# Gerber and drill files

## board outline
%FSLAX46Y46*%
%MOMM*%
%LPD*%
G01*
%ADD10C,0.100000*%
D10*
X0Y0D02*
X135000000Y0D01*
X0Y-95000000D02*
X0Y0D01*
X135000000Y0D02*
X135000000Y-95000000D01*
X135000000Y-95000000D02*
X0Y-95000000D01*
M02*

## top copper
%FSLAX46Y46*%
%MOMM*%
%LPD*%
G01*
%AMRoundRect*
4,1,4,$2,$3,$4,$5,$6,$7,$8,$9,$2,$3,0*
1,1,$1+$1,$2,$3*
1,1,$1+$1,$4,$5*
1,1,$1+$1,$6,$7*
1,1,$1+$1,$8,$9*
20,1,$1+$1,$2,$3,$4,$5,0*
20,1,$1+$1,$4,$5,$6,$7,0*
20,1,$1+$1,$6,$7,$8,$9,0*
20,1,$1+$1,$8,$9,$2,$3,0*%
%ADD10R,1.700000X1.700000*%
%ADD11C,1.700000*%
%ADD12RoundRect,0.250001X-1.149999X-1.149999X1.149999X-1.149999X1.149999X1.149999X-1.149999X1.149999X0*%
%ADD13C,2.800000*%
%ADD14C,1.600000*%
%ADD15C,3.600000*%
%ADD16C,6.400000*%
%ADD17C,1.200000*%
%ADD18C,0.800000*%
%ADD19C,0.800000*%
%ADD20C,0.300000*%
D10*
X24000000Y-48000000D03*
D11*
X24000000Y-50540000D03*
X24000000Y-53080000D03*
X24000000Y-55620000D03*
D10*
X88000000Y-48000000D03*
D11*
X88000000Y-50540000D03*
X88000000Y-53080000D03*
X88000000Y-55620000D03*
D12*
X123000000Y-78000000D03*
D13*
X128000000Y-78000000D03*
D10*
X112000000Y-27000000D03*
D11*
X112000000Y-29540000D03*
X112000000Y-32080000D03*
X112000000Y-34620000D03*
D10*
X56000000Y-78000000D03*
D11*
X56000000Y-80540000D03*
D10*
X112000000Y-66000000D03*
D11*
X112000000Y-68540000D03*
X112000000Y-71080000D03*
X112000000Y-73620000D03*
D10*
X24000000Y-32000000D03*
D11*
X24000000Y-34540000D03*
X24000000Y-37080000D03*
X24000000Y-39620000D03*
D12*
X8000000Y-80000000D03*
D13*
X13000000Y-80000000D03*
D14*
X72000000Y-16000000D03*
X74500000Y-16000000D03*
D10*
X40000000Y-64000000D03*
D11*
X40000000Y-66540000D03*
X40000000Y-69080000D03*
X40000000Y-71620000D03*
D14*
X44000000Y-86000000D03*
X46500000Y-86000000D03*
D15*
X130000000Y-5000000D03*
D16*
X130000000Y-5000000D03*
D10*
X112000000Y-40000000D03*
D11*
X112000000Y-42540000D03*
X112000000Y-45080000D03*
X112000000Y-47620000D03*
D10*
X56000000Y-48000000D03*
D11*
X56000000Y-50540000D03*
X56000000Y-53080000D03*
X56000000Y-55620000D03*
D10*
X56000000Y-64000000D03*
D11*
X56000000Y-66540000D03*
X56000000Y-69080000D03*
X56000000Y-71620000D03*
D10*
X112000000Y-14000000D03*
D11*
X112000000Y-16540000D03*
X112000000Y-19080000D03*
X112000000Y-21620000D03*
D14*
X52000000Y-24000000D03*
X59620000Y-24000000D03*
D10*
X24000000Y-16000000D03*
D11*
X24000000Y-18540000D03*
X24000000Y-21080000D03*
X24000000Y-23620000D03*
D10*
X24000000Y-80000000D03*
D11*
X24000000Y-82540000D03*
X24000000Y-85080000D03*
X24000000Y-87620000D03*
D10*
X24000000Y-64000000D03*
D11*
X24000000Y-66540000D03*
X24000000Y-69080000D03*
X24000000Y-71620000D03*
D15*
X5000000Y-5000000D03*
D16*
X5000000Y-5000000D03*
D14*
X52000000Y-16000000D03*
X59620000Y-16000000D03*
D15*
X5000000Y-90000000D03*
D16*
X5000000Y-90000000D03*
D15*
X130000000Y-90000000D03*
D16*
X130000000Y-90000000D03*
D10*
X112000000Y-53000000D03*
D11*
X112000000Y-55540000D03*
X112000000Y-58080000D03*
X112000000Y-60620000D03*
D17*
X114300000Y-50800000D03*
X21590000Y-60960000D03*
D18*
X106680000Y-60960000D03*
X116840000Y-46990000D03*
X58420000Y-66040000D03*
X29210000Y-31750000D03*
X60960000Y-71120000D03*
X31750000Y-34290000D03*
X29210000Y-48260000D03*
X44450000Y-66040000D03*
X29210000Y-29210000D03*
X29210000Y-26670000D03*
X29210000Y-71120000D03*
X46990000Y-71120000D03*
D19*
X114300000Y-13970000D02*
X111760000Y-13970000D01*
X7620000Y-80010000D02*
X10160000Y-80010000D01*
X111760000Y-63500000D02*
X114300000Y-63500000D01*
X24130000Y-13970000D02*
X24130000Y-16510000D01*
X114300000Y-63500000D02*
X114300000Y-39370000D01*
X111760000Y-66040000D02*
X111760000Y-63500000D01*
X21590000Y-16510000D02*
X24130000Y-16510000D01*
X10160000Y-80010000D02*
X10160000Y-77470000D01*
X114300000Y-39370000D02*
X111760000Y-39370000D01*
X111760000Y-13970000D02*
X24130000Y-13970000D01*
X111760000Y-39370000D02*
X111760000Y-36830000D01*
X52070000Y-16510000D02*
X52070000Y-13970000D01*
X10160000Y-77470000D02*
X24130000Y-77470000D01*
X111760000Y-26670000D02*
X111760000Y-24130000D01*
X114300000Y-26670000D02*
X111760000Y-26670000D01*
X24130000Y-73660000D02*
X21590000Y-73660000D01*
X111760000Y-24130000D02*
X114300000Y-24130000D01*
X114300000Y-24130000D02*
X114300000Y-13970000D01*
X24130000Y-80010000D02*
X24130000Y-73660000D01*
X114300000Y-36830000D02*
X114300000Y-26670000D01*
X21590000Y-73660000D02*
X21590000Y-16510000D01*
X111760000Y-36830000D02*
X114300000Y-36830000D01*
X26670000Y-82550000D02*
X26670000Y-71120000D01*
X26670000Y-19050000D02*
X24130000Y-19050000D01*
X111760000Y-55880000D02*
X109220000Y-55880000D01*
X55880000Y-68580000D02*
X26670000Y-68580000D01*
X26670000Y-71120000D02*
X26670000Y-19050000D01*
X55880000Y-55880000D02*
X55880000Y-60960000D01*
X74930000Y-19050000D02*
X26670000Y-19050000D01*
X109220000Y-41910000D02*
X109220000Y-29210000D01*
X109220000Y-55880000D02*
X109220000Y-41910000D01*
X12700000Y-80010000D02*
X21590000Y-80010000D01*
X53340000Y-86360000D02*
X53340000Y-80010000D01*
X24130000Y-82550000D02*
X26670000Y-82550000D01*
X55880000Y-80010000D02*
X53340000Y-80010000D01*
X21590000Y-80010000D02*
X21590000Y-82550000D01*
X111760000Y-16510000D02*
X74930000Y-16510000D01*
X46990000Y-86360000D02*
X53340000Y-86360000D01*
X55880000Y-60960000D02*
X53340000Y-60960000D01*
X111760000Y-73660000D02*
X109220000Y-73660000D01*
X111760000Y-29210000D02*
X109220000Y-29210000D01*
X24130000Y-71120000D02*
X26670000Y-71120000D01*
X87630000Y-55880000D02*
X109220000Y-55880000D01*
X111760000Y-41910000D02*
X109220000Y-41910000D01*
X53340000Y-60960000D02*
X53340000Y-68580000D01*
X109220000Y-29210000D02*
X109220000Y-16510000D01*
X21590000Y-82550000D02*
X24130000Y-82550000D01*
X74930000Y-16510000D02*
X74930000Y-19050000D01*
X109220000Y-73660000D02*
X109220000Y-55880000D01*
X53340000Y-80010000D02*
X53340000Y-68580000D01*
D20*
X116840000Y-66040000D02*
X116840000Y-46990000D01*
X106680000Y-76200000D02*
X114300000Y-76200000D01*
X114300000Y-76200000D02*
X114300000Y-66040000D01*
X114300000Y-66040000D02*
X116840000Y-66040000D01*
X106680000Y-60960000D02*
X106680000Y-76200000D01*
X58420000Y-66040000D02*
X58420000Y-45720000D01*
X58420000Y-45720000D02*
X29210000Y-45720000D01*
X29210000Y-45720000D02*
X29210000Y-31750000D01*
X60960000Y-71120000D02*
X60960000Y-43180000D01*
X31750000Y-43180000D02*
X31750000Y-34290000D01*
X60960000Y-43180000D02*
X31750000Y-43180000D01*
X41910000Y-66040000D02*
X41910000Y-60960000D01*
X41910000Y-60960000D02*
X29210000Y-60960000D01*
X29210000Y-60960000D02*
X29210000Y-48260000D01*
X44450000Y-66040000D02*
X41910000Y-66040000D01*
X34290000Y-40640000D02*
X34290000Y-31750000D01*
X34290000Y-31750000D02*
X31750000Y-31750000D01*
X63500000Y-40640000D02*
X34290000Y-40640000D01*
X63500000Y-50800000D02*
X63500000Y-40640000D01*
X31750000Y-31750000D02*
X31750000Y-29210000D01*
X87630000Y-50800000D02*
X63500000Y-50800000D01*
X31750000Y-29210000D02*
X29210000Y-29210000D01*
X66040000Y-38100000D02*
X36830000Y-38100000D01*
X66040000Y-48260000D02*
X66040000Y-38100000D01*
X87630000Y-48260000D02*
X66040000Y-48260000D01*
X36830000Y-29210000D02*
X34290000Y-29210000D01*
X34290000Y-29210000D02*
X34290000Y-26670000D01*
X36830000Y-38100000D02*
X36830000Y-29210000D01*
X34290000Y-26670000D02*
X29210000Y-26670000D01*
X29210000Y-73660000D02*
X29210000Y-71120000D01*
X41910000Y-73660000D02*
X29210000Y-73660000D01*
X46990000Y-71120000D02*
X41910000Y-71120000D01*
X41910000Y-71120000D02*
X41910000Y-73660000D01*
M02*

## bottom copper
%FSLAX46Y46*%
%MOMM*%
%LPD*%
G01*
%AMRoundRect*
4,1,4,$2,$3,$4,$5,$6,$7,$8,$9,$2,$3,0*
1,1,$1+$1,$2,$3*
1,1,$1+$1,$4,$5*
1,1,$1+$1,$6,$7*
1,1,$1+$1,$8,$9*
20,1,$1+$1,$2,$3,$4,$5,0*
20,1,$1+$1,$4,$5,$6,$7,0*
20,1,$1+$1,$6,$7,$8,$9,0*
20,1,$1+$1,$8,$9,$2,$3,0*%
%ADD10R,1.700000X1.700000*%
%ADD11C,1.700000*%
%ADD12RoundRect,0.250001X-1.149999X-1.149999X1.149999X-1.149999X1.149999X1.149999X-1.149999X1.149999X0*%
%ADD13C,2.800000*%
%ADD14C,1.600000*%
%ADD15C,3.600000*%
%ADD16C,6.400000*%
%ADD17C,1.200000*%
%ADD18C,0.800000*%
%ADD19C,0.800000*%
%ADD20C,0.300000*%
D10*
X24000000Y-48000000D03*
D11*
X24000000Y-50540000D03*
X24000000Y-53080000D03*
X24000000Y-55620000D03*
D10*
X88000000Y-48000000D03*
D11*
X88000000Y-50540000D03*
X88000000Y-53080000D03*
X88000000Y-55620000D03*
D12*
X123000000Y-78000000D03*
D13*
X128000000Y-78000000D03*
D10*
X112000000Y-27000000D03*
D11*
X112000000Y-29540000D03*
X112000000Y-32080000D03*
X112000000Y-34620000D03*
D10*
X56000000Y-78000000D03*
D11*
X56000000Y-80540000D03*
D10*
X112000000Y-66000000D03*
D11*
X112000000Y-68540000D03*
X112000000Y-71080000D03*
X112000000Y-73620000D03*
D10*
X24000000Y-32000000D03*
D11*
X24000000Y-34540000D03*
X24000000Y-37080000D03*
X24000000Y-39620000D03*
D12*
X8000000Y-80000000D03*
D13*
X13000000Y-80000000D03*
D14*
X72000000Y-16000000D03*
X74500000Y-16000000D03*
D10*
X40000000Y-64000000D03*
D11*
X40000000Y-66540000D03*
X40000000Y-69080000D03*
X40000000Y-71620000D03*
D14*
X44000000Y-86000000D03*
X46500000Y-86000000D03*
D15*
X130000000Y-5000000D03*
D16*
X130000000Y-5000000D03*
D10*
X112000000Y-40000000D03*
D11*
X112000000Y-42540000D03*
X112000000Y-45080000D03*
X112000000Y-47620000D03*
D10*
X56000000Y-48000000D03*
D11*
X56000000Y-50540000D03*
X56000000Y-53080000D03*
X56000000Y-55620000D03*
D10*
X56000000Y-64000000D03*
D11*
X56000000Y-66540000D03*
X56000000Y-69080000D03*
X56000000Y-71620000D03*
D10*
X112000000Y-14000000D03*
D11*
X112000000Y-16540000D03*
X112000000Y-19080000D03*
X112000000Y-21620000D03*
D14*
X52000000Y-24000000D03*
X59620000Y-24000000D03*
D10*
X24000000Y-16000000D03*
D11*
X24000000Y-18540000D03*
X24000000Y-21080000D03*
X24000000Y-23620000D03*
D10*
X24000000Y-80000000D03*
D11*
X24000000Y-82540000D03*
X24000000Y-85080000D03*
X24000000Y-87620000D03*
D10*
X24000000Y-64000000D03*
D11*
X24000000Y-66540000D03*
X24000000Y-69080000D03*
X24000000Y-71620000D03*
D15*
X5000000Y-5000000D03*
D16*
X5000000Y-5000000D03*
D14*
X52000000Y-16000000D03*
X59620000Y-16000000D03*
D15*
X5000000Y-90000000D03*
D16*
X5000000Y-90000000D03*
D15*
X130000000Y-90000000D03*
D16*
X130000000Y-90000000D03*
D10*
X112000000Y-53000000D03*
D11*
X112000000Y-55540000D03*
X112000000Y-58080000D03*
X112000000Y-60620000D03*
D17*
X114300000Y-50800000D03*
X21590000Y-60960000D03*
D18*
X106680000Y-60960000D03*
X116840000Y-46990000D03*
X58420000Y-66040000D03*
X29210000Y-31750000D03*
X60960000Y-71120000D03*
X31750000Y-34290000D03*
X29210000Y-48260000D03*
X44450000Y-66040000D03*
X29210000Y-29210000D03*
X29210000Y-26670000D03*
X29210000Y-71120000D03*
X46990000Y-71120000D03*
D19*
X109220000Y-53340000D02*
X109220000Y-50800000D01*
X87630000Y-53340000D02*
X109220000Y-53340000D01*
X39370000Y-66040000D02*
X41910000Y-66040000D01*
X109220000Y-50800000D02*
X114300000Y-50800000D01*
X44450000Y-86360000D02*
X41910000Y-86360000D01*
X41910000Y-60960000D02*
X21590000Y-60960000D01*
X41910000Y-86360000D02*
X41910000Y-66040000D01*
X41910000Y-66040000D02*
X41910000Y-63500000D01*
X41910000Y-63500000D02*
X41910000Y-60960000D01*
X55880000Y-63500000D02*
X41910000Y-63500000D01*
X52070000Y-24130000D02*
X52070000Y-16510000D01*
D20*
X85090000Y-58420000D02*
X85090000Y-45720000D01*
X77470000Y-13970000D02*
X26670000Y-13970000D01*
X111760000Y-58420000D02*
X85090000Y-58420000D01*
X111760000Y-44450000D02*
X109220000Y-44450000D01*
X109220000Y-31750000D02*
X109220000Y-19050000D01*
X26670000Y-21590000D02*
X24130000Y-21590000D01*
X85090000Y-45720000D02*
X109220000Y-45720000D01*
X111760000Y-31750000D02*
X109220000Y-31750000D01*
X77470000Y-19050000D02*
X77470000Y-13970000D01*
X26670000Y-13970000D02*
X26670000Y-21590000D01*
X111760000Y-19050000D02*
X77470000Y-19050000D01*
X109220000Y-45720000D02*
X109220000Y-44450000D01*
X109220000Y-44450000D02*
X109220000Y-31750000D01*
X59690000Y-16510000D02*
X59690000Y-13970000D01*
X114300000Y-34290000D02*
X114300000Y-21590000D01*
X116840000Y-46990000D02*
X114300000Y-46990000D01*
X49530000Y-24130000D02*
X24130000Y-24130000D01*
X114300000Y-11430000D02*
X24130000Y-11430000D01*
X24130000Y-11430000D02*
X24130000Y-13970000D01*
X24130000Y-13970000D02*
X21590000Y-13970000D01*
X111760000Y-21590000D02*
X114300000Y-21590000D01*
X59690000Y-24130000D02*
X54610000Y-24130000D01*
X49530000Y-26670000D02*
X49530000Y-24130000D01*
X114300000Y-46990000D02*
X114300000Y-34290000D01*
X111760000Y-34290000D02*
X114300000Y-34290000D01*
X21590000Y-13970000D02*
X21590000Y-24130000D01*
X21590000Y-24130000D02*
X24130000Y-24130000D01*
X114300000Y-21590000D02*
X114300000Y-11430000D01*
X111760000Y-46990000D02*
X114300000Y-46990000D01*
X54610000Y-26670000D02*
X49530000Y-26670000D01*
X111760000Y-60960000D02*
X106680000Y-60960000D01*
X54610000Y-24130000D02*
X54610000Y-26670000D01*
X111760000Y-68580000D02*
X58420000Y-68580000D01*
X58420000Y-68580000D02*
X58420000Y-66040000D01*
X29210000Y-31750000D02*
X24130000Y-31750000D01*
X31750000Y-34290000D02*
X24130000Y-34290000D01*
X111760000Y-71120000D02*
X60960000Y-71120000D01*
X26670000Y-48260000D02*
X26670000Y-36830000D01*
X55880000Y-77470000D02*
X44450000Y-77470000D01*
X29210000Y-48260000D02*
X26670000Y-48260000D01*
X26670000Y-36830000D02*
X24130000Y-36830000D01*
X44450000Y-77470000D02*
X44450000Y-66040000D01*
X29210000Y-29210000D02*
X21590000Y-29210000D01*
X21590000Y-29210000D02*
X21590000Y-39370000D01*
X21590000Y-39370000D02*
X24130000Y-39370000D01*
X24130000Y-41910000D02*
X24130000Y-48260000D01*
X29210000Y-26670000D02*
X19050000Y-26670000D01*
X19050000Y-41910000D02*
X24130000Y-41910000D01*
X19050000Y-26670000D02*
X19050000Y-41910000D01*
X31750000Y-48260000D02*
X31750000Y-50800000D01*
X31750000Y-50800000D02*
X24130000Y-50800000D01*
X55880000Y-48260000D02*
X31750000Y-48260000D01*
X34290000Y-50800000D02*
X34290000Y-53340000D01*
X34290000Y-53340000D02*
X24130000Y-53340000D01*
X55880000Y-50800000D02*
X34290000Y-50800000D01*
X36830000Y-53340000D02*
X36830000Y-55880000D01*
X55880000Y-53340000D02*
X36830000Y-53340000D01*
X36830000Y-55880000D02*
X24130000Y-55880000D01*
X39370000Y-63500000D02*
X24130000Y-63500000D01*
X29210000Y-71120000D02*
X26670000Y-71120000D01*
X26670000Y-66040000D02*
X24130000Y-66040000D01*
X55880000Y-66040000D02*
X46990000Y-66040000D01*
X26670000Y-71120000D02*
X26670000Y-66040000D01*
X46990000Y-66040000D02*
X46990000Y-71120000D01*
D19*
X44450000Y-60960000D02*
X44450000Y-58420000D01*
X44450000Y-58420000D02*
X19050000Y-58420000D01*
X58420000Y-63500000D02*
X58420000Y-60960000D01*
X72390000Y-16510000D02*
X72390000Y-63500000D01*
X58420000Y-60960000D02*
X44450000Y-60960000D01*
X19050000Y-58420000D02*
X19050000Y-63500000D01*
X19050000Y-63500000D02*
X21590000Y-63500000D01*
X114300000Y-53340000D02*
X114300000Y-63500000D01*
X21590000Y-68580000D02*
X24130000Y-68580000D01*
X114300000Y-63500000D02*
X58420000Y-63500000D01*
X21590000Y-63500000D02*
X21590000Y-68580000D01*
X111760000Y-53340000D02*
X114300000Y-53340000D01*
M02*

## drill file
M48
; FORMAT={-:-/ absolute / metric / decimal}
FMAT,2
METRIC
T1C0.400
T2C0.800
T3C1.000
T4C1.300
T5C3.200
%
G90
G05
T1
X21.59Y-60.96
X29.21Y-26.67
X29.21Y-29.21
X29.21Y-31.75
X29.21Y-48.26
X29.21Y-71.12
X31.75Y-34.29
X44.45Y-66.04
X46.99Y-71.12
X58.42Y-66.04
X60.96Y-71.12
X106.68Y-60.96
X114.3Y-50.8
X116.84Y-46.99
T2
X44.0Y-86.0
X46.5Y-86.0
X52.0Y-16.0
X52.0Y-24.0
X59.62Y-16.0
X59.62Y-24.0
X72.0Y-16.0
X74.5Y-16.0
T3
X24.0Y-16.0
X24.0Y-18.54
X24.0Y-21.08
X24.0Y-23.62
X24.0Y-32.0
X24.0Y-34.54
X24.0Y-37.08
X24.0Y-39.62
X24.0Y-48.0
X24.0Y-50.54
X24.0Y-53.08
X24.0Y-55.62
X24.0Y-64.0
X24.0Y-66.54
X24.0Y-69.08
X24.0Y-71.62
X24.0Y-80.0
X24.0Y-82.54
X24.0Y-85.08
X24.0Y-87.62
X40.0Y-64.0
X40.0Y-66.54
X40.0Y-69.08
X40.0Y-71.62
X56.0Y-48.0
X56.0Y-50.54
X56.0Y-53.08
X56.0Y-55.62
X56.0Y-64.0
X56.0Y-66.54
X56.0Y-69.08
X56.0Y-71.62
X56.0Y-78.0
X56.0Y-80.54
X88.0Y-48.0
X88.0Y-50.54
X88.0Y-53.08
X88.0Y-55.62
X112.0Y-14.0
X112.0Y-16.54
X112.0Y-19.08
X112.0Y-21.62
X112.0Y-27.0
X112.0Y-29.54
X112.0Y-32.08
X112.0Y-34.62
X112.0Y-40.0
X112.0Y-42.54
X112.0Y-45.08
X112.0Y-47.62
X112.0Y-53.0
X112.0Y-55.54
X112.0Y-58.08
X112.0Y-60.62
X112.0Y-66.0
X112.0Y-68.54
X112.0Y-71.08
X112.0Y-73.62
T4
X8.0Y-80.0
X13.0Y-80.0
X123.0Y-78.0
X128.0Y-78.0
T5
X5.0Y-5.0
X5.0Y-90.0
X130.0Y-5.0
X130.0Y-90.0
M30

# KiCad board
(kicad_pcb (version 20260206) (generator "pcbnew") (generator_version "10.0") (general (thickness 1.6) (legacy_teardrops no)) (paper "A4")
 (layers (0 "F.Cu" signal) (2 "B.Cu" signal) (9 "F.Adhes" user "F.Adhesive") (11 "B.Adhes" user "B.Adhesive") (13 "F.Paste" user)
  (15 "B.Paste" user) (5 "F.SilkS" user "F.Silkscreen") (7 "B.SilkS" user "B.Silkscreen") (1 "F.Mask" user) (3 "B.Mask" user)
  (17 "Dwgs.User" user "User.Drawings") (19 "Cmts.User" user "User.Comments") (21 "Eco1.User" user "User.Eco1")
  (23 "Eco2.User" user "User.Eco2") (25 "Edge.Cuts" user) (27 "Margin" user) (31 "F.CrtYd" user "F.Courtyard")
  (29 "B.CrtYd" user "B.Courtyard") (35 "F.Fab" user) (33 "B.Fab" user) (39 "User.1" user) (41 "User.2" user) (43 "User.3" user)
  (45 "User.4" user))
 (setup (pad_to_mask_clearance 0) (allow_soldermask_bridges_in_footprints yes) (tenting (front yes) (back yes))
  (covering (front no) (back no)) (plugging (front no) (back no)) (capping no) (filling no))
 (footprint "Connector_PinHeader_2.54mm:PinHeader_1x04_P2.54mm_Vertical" (layer "F.Cu") (at 24 48)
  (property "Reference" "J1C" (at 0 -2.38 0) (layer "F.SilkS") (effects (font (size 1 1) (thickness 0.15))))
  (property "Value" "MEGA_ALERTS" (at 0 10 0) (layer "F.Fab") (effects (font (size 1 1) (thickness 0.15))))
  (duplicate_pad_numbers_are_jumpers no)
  (pad "1" thru_hole rect (at 0 0) (size 1.7 1.7) (drill 1) (layers "*.Cu" "*.Mask") (remove_unused_layers no) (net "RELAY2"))
  (pad "2" thru_hole circle (at 0 2.54) (size 1.7 1.7) (drill 1) (layers "*.Cu" "*.Mask") (remove_unused_layers no) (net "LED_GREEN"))
  (pad "3" thru_hole circle (at 0 5.08) (size 1.7 1.7) (drill 1) (layers "*.Cu" "*.Mask") (remove_unused_layers no) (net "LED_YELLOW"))
  (pad "4" thru_hole circle (at 0 7.62) (size 1.7 1.7) (drill 1) (layers "*.Cu" "*.Mask") (remove_unused_layers no) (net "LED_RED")))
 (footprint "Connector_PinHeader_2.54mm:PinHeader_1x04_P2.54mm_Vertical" (layer "F.Cu") (at 88 48)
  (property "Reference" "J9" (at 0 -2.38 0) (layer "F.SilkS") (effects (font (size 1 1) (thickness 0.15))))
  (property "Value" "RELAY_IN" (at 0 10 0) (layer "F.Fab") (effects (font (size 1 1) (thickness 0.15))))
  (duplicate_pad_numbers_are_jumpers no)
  (pad "1" thru_hole rect (at 0 0) (size 1.7 1.7) (drill 1) (layers "*.Cu" "*.Mask") (remove_unused_layers no) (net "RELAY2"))
  (pad "2" thru_hole circle (at 0 2.54) (size 1.7 1.7) (drill 1) (layers "*.Cu" "*.Mask") (remove_unused_layers no) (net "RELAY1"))
  (pad "3" thru_hole circle (at 0 5.08) (size 1.7 1.7) (drill 1) (layers "*.Cu" "*.Mask") (remove_unused_layers no) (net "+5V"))
  (pad "4" thru_hole circle (at 0 7.62) (size 1.7 1.7) (drill 1) (layers "*.Cu" "*.Mask") (remove_unused_layers no) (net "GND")))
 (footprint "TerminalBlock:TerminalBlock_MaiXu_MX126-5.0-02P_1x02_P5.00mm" (layer "F.Cu") (at 123 78)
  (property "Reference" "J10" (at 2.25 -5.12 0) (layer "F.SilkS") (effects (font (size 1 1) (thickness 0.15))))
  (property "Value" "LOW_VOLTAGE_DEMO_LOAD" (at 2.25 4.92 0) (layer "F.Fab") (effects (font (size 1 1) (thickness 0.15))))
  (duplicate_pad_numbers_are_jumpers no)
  (pad "1" thru_hole roundrect (at 0 0) (size 2.8 2.8) (drill 1.3) (layers "*.Cu" "*.Mask") (remove_unused_layers no)
   (roundrect_rratio 0.089286) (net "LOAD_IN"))
  (pad "2" thru_hole circle (at 5 0) (size 2.8 2.8) (drill 1.3) (layers "*.Cu" "*.Mask") (remove_unused_layers no) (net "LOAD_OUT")))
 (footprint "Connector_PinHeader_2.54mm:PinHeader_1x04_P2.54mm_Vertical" (layer "F.Cu") (at 112 27)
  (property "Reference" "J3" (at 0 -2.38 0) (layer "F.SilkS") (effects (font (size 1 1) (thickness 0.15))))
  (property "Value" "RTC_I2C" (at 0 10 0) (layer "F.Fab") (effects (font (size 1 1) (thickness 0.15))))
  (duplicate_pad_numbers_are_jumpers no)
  (pad "1" thru_hole rect (at 0 0) (size 1.7 1.7) (drill 1) (layers "*.Cu" "*.Mask") (remove_unused_layers no) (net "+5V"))
  (pad "2" thru_hole circle (at 0 2.54) (size 1.7 1.7) (drill 1) (layers "*.Cu" "*.Mask") (remove_unused_layers no) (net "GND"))
  (pad "3" thru_hole circle (at 0 5.08) (size 1.7 1.7) (drill 1) (layers "*.Cu" "*.Mask") (remove_unused_layers no) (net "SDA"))
  (pad "4" thru_hole circle (at 0 7.62) (size 1.7 1.7) (drill 1) (layers "*.Cu" "*.Mask") (remove_unused_layers no) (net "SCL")))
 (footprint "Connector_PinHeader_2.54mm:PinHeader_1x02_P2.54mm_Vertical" (layer "F.Cu") (at 56 78)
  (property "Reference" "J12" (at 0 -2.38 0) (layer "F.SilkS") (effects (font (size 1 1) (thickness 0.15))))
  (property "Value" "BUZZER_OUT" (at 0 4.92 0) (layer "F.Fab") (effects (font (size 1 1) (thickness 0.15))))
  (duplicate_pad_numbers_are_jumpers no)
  (pad "1" thru_hole rect (at 0 0) (size 1.7 1.7) (drill 1) (layers "*.Cu" "*.Mask") (remove_unused_layers no) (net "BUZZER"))
  (pad "2" thru_hole circle (at 0 2.54) (size 1.7 1.7) (drill 1) (layers "*.Cu" "*.Mask") (remove_unused_layers no) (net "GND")))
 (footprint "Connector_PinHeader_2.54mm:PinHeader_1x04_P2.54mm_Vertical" (layer "F.Cu") (at 112 66)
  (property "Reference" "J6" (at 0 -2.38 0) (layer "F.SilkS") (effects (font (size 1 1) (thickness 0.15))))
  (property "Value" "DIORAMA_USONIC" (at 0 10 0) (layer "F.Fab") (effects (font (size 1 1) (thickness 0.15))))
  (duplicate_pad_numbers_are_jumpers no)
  (pad "1" thru_hole rect (at 0 0) (size 1.7 1.7) (drill 1) (layers "*.Cu" "*.Mask") (remove_unused_layers no) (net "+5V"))
  (pad "2" thru_hole circle (at 0 2.54) (size 1.7 1.7) (drill 1) (layers "*.Cu" "*.Mask") (remove_unused_layers no) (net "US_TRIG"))
  (pad "3" thru_hole circle (at 0 5.08) (size 1.7 1.7) (drill 1) (layers "*.Cu" "*.Mask") (remove_unused_layers no) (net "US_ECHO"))
  (pad "4" thru_hole circle (at 0 7.62) (size 1.7 1.7) (drill 1) (layers "*.Cu" "*.Mask") (remove_unused_layers no) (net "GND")))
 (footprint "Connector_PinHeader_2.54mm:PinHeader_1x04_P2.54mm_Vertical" (layer "F.Cu") (at 24 32)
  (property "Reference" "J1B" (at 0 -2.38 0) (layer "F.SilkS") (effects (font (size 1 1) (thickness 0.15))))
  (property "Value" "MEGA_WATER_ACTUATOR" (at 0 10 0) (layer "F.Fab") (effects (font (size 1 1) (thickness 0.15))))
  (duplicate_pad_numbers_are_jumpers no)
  (pad "1" thru_hole rect (at 0 0) (size 1.7 1.7) (drill 1) (layers "*.Cu" "*.Mask") (remove_unused_layers no) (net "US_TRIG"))
  (pad "2" thru_hole circle (at 0 2.54) (size 1.7 1.7) (drill 1) (layers "*.Cu" "*.Mask") (remove_unused_layers no) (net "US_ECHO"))
  (pad "3" thru_hole circle (at 0 5.08) (size 1.7 1.7) (drill 1) (layers "*.Cu" "*.Mask") (remove_unused_layers no) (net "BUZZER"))
  (pad "4" thru_hole circle (at 0 7.62) (size 1.7 1.7) (drill 1) (layers "*.Cu" "*.Mask") (remove_unused_layers no) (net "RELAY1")))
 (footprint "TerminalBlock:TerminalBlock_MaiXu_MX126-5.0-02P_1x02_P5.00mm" (layer "F.Cu") (at 8 80)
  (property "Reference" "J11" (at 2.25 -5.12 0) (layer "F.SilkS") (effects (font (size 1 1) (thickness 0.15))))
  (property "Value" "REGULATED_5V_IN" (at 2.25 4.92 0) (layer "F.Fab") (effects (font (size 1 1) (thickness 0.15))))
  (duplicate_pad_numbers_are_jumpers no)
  (pad "1" thru_hole roundrect (at 0 0) (size 2.8 2.8) (drill 1.3) (layers "*.Cu" "*.Mask") (remove_unused_layers no)
   (roundrect_rratio 0.089286) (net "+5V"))
  (pad "2" thru_hole circle (at 5 0) (size 2.8 2.8) (drill 1.3) (layers "*.Cu" "*.Mask") (remove_unused_layers no) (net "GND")))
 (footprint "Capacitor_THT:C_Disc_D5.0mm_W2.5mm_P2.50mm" (layer "F.Cu") (at 72 16)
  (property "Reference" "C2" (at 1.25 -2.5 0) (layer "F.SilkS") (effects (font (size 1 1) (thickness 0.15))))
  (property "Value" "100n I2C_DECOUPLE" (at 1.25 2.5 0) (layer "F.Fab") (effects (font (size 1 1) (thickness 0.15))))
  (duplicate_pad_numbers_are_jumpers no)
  (pad "1" thru_hole circle (at 0 0) (size 1.6 1.6) (drill 0.8) (layers "*.Cu" "*.Mask") (remove_unused_layers no) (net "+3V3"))
  (pad "2" thru_hole circle (at 2.5 0) (size 1.6 1.6) (drill 0.8) (layers "*.Cu" "*.Mask") (remove_unused_layers no) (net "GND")))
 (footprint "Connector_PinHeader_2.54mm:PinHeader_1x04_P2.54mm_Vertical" (layer "F.Cu") (at 40 64)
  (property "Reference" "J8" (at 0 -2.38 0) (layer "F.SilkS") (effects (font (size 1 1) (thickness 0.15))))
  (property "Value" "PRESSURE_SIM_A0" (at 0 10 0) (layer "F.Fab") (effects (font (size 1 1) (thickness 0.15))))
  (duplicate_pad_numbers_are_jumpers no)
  (pad "1" thru_hole rect (at 0 0) (size 1.7 1.7) (drill 1) (layers "*.Cu" "*.Mask") (remove_unused_layers no) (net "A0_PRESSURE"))
  (pad "2" thru_hole circle (at 0 2.54) (size 1.7 1.7) (drill 1) (layers "*.Cu" "*.Mask") (remove_unused_layers no) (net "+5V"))
  (pad "3" thru_hole circle (at 0 5.08) (size 1.7 1.7) (drill 1) (layers "*.Cu" "*.Mask") (remove_unused_layers no) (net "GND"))
  (pad "4" thru_hole circle (at 0 7.62) (size 1.7 1.7) (drill 1) (layers "*.Cu" "*.Mask") (remove_unused_layers no)))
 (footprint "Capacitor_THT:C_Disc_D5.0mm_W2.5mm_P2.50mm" (layer "F.Cu") (at 44 86)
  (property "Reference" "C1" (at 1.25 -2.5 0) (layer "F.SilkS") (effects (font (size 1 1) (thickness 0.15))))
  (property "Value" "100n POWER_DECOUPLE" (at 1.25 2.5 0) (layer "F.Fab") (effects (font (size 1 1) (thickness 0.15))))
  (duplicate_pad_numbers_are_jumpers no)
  (pad "1" thru_hole circle (at 0 0) (size 1.6 1.6) (drill 0.8) (layers "*.Cu" "*.Mask") (remove_unused_layers no) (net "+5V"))
  (pad "2" thru_hole circle (at 2.5 0) (size 1.6 1.6) (drill 0.8) (layers "*.Cu" "*.Mask") (remove_unused_layers no) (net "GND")))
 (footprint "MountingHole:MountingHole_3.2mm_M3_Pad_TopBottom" (layer "F.Cu") (at 130 5)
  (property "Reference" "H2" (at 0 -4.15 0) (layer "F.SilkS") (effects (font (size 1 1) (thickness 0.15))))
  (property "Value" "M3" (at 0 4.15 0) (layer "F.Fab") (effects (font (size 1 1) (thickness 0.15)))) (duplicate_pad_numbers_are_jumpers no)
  (pad "1" thru_hole circle (at 0 0) (size 3.6 3.6) (drill 3.2) (layers "*.Cu" "*.Mask") (remove_unused_layers no) (zone_connect 2))
  (pad "1" connect circle (at 0 0) (size 6.4 6.4) (layers "F.Cu" "F.Mask") (zone_connect 2))
  (pad "1" connect circle (at 0 0) (size 6.4 6.4) (layers "B.Cu" "B.Mask") (zone_connect 2)))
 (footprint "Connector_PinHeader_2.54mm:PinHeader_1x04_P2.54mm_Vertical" (layer "F.Cu") (at 112 40)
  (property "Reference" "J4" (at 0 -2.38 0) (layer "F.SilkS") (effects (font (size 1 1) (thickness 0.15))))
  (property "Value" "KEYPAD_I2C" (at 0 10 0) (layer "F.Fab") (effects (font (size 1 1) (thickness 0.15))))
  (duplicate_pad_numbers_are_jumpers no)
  (pad "1" thru_hole rect (at 0 0) (size 1.7 1.7) (drill 1) (layers "*.Cu" "*.Mask") (remove_unused_layers no) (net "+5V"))
  (pad "2" thru_hole circle (at 0 2.54) (size 1.7 1.7) (drill 1) (layers "*.Cu" "*.Mask") (remove_unused_layers no) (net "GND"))
  (pad "3" thru_hole circle (at 0 5.08) (size 1.7 1.7) (drill 1) (layers "*.Cu" "*.Mask") (remove_unused_layers no) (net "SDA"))
  (pad "4" thru_hole circle (at 0 7.62) (size 1.7 1.7) (drill 1) (layers "*.Cu" "*.Mask") (remove_unused_layers no) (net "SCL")))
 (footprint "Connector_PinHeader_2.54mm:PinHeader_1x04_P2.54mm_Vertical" (layer "F.Cu") (at 56 48)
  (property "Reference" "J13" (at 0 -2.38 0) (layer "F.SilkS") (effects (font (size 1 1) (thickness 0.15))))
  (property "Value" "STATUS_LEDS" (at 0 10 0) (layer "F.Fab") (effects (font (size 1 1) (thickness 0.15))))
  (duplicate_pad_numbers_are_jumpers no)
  (pad "1" thru_hole rect (at 0 0) (size 1.7 1.7) (drill 1) (layers "*.Cu" "*.Mask") (remove_unused_layers no) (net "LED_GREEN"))
  (pad "2" thru_hole circle (at 0 2.54) (size 1.7 1.7) (drill 1) (layers "*.Cu" "*.Mask") (remove_unused_layers no) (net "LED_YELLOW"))
  (pad "3" thru_hole circle (at 0 5.08) (size 1.7 1.7) (drill 1) (layers "*.Cu" "*.Mask") (remove_unused_layers no) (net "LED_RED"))
  (pad "4" thru_hole circle (at 0 7.62) (size 1.7 1.7) (drill 1) (layers "*.Cu" "*.Mask") (remove_unused_layers no) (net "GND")))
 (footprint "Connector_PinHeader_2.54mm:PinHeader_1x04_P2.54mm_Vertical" (layer "F.Cu") (at 56 64)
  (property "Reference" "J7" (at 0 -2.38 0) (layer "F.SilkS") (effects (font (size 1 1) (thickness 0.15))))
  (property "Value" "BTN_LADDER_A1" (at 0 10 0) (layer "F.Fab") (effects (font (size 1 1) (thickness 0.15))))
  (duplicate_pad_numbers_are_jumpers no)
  (pad "1" thru_hole rect (at 0 0) (size 1.7 1.7) (drill 1) (layers "*.Cu" "*.Mask") (remove_unused_layers no) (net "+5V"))
  (pad "2" thru_hole circle (at 0 2.54) (size 1.7 1.7) (drill 1) (layers "*.Cu" "*.Mask") (remove_unused_layers no) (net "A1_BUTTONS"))
  (pad "3" thru_hole circle (at 0 5.08) (size 1.7 1.7) (drill 1) (layers "*.Cu" "*.Mask") (remove_unused_layers no) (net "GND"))
  (pad "4" thru_hole circle (at 0 7.62) (size 1.7 1.7) (drill 1) (layers "*.Cu" "*.Mask") (remove_unused_layers no)))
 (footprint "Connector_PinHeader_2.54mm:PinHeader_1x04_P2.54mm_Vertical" (layer "F.Cu") (at 112 14)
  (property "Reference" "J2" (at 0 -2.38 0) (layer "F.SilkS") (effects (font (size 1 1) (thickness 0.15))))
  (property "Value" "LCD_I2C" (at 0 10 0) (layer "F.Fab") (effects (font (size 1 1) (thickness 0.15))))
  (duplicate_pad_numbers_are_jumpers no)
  (pad "1" thru_hole rect (at 0 0) (size 1.7 1.7) (drill 1) (layers "*.Cu" "*.Mask") (remove_unused_layers no) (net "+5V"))
  (pad "2" thru_hole circle (at 0 2.54) (size 1.7 1.7) (drill 1) (layers "*.Cu" "*.Mask") (remove_unused_layers no) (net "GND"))
  (pad "3" thru_hole circle (at 0 5.08) (size 1.7 1.7) (drill 1) (layers "*.Cu" "*.Mask") (remove_unused_layers no) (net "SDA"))
  (pad "4" thru_hole circle (at 0 7.62) (size 1.7 1.7) (drill 1) (layers "*.Cu" "*.Mask") (remove_unused_layers no) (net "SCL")))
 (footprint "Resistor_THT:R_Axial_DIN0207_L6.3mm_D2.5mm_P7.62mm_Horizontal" (layer "F.Cu") (at 52 24)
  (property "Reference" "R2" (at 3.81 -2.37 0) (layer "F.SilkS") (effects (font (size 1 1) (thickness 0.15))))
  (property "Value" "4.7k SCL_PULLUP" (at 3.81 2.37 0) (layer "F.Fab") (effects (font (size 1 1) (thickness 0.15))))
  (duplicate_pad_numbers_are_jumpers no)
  (pad "1" thru_hole circle (at 0 0) (size 1.6 1.6) (drill 0.8) (layers "*.Cu" "*.Mask") (remove_unused_layers no) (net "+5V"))
  (pad "2" thru_hole circle (at 7.62 0) (size 1.6 1.6) (drill 0.8) (layers "*.Cu" "*.Mask") (remove_unused_layers no) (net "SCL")))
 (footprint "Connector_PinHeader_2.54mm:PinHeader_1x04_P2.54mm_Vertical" (layer "F.Cu") (at 24 16)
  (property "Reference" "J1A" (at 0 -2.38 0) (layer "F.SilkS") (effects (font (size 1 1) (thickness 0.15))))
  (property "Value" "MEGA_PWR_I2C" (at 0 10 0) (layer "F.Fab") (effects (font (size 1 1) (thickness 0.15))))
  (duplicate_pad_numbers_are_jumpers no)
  (pad "1" thru_hole rect (at 0 0) (size 1.7 1.7) (drill 1) (layers "*.Cu" "*.Mask") (remove_unused_layers no) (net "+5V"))
  (pad "2" thru_hole circle (at 0 2.54) (size 1.7 1.7) (drill 1) (layers "*.Cu" "*.Mask") (remove_unused_layers no) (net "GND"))
  (pad "3" thru_hole circle (at 0 5.08) (size 1.7 1.7) (drill 1) (layers "*.Cu" "*.Mask") (remove_unused_layers no) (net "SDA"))
  (pad "4" thru_hole circle (at 0 7.62) (size 1.7 1.7) (drill 1) (layers "*.Cu" "*.Mask") (remove_unused_layers no) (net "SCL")))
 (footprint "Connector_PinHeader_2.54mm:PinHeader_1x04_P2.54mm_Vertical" (layer "F.Cu") (at 24 80)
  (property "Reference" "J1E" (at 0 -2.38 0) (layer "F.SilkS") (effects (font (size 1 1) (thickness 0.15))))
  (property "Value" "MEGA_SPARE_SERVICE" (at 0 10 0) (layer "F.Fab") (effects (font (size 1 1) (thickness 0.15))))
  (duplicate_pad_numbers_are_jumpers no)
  (pad "1" thru_hole rect (at 0 0) (size 1.7 1.7) (drill 1) (layers "*.Cu" "*.Mask") (remove_unused_layers no) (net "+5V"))
  (pad "2" thru_hole circle (at 0 2.54) (size 1.7 1.7) (drill 1) (layers "*.Cu" "*.Mask") (remove_unused_layers no) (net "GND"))
  (pad "3" thru_hole circle (at 0 5.08) (size 1.7 1.7) (drill 1) (layers "*.Cu" "*.Mask") (remove_unused_layers no))
  (pad "4" thru_hole circle (at 0 7.62) (size 1.7 1.7) (drill 1) (layers "*.Cu" "*.Mask") (remove_unused_layers no)))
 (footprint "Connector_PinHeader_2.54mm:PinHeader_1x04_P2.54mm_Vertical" (layer "F.Cu") (at 24 64)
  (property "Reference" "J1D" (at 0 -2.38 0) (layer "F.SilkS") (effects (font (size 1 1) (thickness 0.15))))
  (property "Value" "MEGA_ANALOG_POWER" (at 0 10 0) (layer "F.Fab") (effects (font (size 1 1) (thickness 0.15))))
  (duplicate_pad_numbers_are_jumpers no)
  (pad "1" thru_hole rect (at 0 0) (size 1.7 1.7) (drill 1) (layers "*.Cu" "*.Mask") (remove_unused_layers no) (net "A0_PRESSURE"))
  (pad "2" thru_hole circle (at 0 2.54) (size 1.7 1.7) (drill 1) (layers "*.Cu" "*.Mask") (remove_unused_layers no) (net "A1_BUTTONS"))
  (pad "3" thru_hole circle (at 0 5.08) (size 1.7 1.7) (drill 1) (layers "*.Cu" "*.Mask") (remove_unused_layers no) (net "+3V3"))
  (pad "4" thru_hole circle (at 0 7.62) (size 1.7 1.7) (drill 1) (layers "*.Cu" "*.Mask") (remove_unused_layers no) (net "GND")))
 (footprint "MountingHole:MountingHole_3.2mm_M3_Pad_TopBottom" (layer "F.Cu") (at 5 5)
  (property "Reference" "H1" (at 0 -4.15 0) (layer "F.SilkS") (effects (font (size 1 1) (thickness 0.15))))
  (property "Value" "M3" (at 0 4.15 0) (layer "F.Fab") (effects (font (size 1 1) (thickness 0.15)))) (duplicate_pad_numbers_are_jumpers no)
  (pad "1" thru_hole circle (at 0 0) (size 3.6 3.6) (drill 3.2) (layers "*.Cu" "*.Mask") (remove_unused_layers no) (zone_connect 2))
  (pad "1" connect circle (at 0 0) (size 6.4 6.4) (layers "F.Cu" "F.Mask") (zone_connect 2))
  (pad "1" connect circle (at 0 0) (size 6.4 6.4) (layers "B.Cu" "B.Mask") (zone_connect 2)))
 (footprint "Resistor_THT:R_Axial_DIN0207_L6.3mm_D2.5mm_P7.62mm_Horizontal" (layer "F.Cu") (at 52 16)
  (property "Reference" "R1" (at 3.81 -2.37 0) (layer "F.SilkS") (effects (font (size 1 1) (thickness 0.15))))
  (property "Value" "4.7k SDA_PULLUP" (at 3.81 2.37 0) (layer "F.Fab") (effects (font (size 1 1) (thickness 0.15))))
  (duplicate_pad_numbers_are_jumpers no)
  (pad "1" thru_hole circle (at 0 0) (size 1.6 1.6) (drill 0.8) (layers "*.Cu" "*.Mask") (remove_unused_layers no) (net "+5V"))
  (pad "2" thru_hole circle (at 7.62 0) (size 1.6 1.6) (drill 0.8) (layers "*.Cu" "*.Mask") (remove_unused_layers no) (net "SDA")))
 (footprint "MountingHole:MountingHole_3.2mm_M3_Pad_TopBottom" (layer "F.Cu") (at 5 90)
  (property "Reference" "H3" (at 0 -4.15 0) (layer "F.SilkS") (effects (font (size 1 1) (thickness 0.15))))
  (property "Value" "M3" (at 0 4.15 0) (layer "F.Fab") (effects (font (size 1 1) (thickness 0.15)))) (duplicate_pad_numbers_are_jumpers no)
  (pad "1" thru_hole circle (at 0 0) (size 3.6 3.6) (drill 3.2) (layers "*.Cu" "*.Mask") (remove_unused_layers no) (zone_connect 2))
  (pad "1" connect circle (at 0 0) (size 6.4 6.4) (layers "F.Cu" "F.Mask") (zone_connect 2))
  (pad "1" connect circle (at 0 0) (size 6.4 6.4) (layers "B.Cu" "B.Mask") (zone_connect 2)))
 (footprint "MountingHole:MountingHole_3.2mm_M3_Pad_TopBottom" (layer "F.Cu") (at 130 90)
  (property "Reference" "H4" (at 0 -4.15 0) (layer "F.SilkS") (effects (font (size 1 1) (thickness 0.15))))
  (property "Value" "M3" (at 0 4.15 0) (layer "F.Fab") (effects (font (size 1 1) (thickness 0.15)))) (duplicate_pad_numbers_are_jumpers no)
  (pad "1" thru_hole circle (at 0 0) (size 3.6 3.6) (drill 3.2) (layers "*.Cu" "*.Mask") (remove_unused_layers no) (zone_connect 2))
  (pad "1" connect circle (at 0 0) (size 6.4 6.4) (layers "F.Cu" "F.Mask") (zone_connect 2))
  (pad "1" connect circle (at 0 0) (size 6.4 6.4) (layers "B.Cu" "B.Mask") (zone_connect 2)))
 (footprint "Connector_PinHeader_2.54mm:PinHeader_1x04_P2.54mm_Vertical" (layer "F.Cu") (at 112 53)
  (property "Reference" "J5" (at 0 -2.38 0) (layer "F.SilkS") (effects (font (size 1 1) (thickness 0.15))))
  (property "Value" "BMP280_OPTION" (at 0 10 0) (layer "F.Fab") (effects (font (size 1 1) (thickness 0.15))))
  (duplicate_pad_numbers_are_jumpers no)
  (pad "1" thru_hole rect (at 0 0) (size 1.7 1.7) (drill 1) (layers "*.Cu" "*.Mask") (remove_unused_layers no) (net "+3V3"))
  (pad "2" thru_hole circle (at 0 2.54) (size 1.7 1.7) (drill 1) (layers "*.Cu" "*.Mask") (remove_unused_layers no) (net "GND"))
  (pad "3" thru_hole circle (at 0 5.08) (size 1.7 1.7) (drill 1) (layers "*.Cu" "*.Mask") (remove_unused_layers no) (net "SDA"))
  (pad "4" thru_hole circle (at 0 7.62) (size 1.7 1.7) (drill 1) (layers "*.Cu" "*.Mask") (remove_unused_layers no) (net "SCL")))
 (gr_line (start 0 0) (end 135 0) (stroke (width 0.1) (type default)) (layer "Edge.Cuts"))
 (gr_line (start 0 95) (end 0 0) (stroke (width 0.1) (type default)) (layer "Edge.Cuts"))
 (gr_line (start 135 0) (end 135 95) (stroke (width 0.1) (type default)) (layer "Edge.Cuts"))
 (gr_line (start 135 95) (end 0 95) (stroke (width 0.1) (type default)) (layer "Edge.Cuts"))
 (segment (start 114.3 13.97) (end 111.76 13.97) (width 0.8) (layer "F.Cu") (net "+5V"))
 (segment (start 7.62 80.01) (end 10.16 80.01) (width 0.8) (layer "F.Cu") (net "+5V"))
 (segment (start 111.76 63.5) (end 114.3 63.5) (width 0.8) (layer "F.Cu") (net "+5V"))
 (segment (start 24.13 13.97) (end 24.13 16.51) (width 0.8) (layer "F.Cu") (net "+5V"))
 (segment (start 114.3 63.5) (end 114.3 39.37) (width 0.8) (layer "F.Cu") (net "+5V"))
 (segment (start 111.76 66.04) (end 111.76 63.5) (width 0.8) (layer "F.Cu") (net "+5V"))
 (segment (start 21.59 16.51) (end 24.13 16.51) (width 0.8) (layer "F.Cu") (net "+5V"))
 (segment (start 10.16 80.01) (end 10.16 77.47) (width 0.8) (layer "F.Cu") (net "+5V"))
 (segment (start 114.3 39.37) (end 111.76 39.37) (width 0.8) (layer "F.Cu") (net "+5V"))
 (segment (start 111.76 13.97) (end 24.13 13.97) (width 0.8) (layer "F.Cu") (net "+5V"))
 (segment (start 111.76 39.37) (end 111.76 36.83) (width 0.8) (layer "F.Cu") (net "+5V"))
 (segment (start 52.07 16.51) (end 52.07 13.97) (width 0.8) (layer "F.Cu") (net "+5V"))
 (segment (start 10.16 77.47) (end 24.13 77.47) (width 0.8) (layer "F.Cu") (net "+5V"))
 (segment (start 111.76 26.67) (end 111.76 24.13) (width 0.8) (layer "F.Cu") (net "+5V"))
 (segment (start 114.3 26.67) (end 111.76 26.67) (width 0.8) (layer "F.Cu") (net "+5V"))
 (segment (start 24.13 73.66) (end 21.59 73.66) (width 0.8) (layer "F.Cu") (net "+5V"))
 (segment (start 111.76 24.13) (end 114.3 24.13) (width 0.8) (layer "F.Cu") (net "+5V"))
 (segment (start 114.3 24.13) (end 114.3 13.97) (width 0.8) (layer "F.Cu") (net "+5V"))
 (segment (start 24.13 80.01) (end 24.13 73.66) (width 0.8) (layer "F.Cu") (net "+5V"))
 (segment (start 114.3 36.83) (end 114.3 26.67) (width 0.8) (layer "F.Cu") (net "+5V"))
 (segment (start 21.59 73.66) (end 21.59 16.51) (width 0.8) (layer "F.Cu") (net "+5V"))
 (segment (start 111.76 36.83) (end 114.3 36.83) (width 0.8) (layer "F.Cu") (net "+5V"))
 (via (at 114.3 50.8) (size 1.2) (drill 0.4) (layers "F.Cu" "B.Cu") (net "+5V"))
 (via (at 21.59 60.96) (size 1.2) (drill 0.4) (layers "F.Cu" "B.Cu") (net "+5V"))
 (segment (start 109.22 53.34) (end 109.22 50.8) (width 0.8) (layer "B.Cu") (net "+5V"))
 (segment (start 87.63 53.34) (end 109.22 53.34) (width 0.8) (layer "B.Cu") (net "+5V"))
 (segment (start 39.37 66.04) (end 41.91 66.04) (width 0.8) (layer "B.Cu") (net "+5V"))
 (segment (start 109.22 50.8) (end 114.3 50.8) (width 0.8) (layer "B.Cu") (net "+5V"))
 (segment (start 44.45 86.36) (end 41.91 86.36) (width 0.8) (layer "B.Cu") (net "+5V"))
 (segment (start 41.91 60.96) (end 21.59 60.96) (width 0.8) (layer "B.Cu") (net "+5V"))
 (segment (start 41.91 86.36) (end 41.91 66.04) (width 0.8) (layer "B.Cu") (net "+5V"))
 (segment (start 41.91 66.04) (end 41.91 63.5) (width 0.8) (layer "B.Cu") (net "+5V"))
 (segment (start 41.91 63.5) (end 41.91 60.96) (width 0.8) (layer "B.Cu") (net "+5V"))
 (segment (start 55.88 63.5) (end 41.91 63.5) (width 0.8) (layer "B.Cu") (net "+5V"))
 (segment (start 52.07 24.13) (end 52.07 16.51) (width 0.8) (layer "B.Cu") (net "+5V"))
 (segment (start 26.67 82.55) (end 26.67 71.12) (width 0.8) (layer "F.Cu") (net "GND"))
 (segment (start 26.67 19.05) (end 24.13 19.05) (width 0.8) (layer "F.Cu") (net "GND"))
 (segment (start 111.76 55.88) (end 109.22 55.88) (width 0.8) (layer "F.Cu") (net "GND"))
 (segment (start 55.88 68.58) (end 26.67 68.58) (width 0.8) (layer "F.Cu") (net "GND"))
 (segment (start 26.67 71.12) (end 26.67 19.05) (width 0.8) (layer "F.Cu") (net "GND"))
 (segment (start 55.88 55.88) (end 55.88 60.96) (width 0.8) (layer "F.Cu") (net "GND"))
 (segment (start 74.93 19.05) (end 26.67 19.05) (width 0.8) (layer "F.Cu") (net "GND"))
 (segment (start 109.22 41.91) (end 109.22 29.21) (width 0.8) (layer "F.Cu") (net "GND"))
 (segment (start 109.22 55.88) (end 109.22 41.91) (width 0.8) (layer "F.Cu") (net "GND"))
 (segment (start 12.7 80.01) (end 21.59 80.01) (width 0.8) (layer "F.Cu") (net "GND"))
 (segment (start 53.34 86.36) (end 53.34 80.01) (width 0.8) (layer "F.Cu") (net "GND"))
 (segment (start 24.13 82.55) (end 26.67 82.55) (width 0.8) (layer "F.Cu") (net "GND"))
 (segment (start 55.88 80.01) (end 53.34 80.01) (width 0.8) (layer "F.Cu") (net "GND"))
 (segment (start 21.59 80.01) (end 21.59 82.55) (width 0.8) (layer "F.Cu") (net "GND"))
 (segment (start 111.76 16.51) (end 74.93 16.51) (width 0.8) (layer "F.Cu") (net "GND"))
 (segment (start 46.99 86.36) (end 53.34 86.36) (width 0.8) (layer "F.Cu") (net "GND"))
 (segment (start 55.88 60.96) (end 53.34 60.96) (width 0.8) (layer "F.Cu") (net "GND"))
 (segment (start 111.76 73.66) (end 109.22 73.66) (width 0.8) (layer "F.Cu") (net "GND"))
 (segment (start 111.76 29.21) (end 109.22 29.21) (width 0.8) (layer "F.Cu") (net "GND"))
 (segment (start 24.13 71.12) (end 26.67 71.12) (width 0.8) (layer "F.Cu") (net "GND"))
 (segment (start 87.63 55.88) (end 109.22 55.88) (width 0.8) (layer "F.Cu") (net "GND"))
 (segment (start 111.76 41.91) (end 109.22 41.91) (width 0.8) (layer "F.Cu") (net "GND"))
 (segment (start 53.34 60.96) (end 53.34 68.58) (width 0.8) (layer "F.Cu") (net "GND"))
 (segment (start 109.22 29.21) (end 109.22 16.51) (width 0.8) (layer "F.Cu") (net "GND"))
 (segment (start 21.59 82.55) (end 24.13 82.55) (width 0.8) (layer "F.Cu") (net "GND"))
 (segment (start 74.93 16.51) (end 74.93 19.05) (width 0.8) (layer "F.Cu") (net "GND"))
 (segment (start 109.22 73.66) (end 109.22 55.88) (width 0.8) (layer "F.Cu") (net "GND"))
 (segment (start 53.34 80.01) (end 53.34 68.58) (width 0.8) (layer "F.Cu") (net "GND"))
 (segment (start 85.09 58.42) (end 85.09 45.72) (width 0.3) (layer "B.Cu") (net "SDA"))
 (segment (start 77.47 13.97) (end 26.67 13.97) (width 0.3) (layer "B.Cu") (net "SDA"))
 (segment (start 111.76 58.42) (end 85.09 58.42) (width 0.3) (layer "B.Cu") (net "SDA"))
 (segment (start 111.76 44.45) (end 109.22 44.45) (width 0.3) (layer "B.Cu") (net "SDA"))
 (segment (start 109.22 31.75) (end 109.22 19.05) (width 0.3) (layer "B.Cu") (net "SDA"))
 (segment (start 26.67 21.59) (end 24.13 21.59) (width 0.3) (layer "B.Cu") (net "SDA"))
 (segment (start 85.09 45.72) (end 109.22 45.72) (width 0.3) (layer "B.Cu") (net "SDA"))
 (segment (start 111.76 31.75) (end 109.22 31.75) (width 0.3) (layer "B.Cu") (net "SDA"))
 (segment (start 77.47 19.05) (end 77.47 13.97) (width 0.3) (layer "B.Cu") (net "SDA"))
 (segment (start 26.67 13.97) (end 26.67 21.59) (width 0.3) (layer "B.Cu") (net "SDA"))
 (segment (start 111.76 19.05) (end 77.47 19.05) (width 0.3) (layer "B.Cu") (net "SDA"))
 (segment (start 109.22 45.72) (end 109.22 44.45) (width 0.3) (layer "B.Cu") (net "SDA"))
 (segment (start 109.22 44.45) (end 109.22 31.75) (width 0.3) (layer "B.Cu") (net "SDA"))
 (segment (start 59.69 16.51) (end 59.69 13.97) (width 0.3) (layer "B.Cu") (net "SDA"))
 (segment (start 116.84 66.04) (end 116.84 46.99) (width 0.3) (layer "F.Cu") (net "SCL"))
 (segment (start 106.68 76.2) (end 114.3 76.2) (width 0.3) (layer "F.Cu") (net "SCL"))
 (segment (start 114.3 76.2) (end 114.3 66.04) (width 0.3) (layer "F.Cu") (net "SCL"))
 (segment (start 114.3 66.04) (end 116.84 66.04) (width 0.3) (layer "F.Cu") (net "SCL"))
 (segment (start 106.68 60.96) (end 106.68 76.2) (width 0.3) (layer "F.Cu") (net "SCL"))
 (via (at 106.68 60.96) (size 0.8) (drill 0.4) (layers "F.Cu" "B.Cu") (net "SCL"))
 (via (at 116.84 46.99) (size 0.8) (drill 0.4) (layers "F.Cu" "B.Cu") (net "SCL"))
 (segment (start 114.3 34.29) (end 114.3 21.59) (width 0.3) (layer "B.Cu") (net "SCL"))
 (segment (start 116.84 46.99) (end 114.3 46.99) (width 0.3) (layer "B.Cu") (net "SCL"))
 (segment (start 49.53 24.13) (end 24.13 24.13) (width 0.3) (layer "B.Cu") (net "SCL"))
 (segment (start 114.3 11.43) (end 24.13 11.43) (width 0.3) (layer "B.Cu") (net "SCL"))
 (segment (start 24.13 11.43) (end 24.13 13.97) (width 0.3) (layer "B.Cu") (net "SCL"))
 (segment (start 24.13 13.97) (end 21.59 13.97) (width 0.3) (layer "B.Cu") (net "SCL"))
 (segment (start 111.76 21.59) (end 114.3 21.59) (width 0.3) (layer "B.Cu") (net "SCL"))
 (segment (start 59.69 24.13) (end 54.61 24.13) (width 0.3) (layer "B.Cu") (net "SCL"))
 (segment (start 49.53 26.67) (end 49.53 24.13) (width 0.3) (layer "B.Cu") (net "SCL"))
 (segment (start 114.3 46.99) (end 114.3 34.29) (width 0.3) (layer "B.Cu") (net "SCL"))
 (segment (start 111.76 34.29) (end 114.3 34.29) (width 0.3) (layer "B.Cu") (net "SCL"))
 (segment (start 21.59 13.97) (end 21.59 24.13) (width 0.3) (layer "B.Cu") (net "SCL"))
 (segment (start 21.59 24.13) (end 24.13 24.13) (width 0.3) (layer "B.Cu") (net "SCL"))
 (segment (start 114.3 21.59) (end 114.3 11.43) (width 0.3) (layer "B.Cu") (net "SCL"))
 (segment (start 111.76 46.99) (end 114.3 46.99) (width 0.3) (layer "B.Cu") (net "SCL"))
 (segment (start 54.61 26.67) (end 49.53 26.67) (width 0.3) (layer "B.Cu") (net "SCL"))
 (segment (start 111.76 60.96) (end 106.68 60.96) (width 0.3) (layer "B.Cu") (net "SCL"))
 (segment (start 54.61 24.13) (end 54.61 26.67) (width 0.3) (layer "B.Cu") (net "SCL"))
 (segment (start 58.42 66.04) (end 58.42 45.72) (width 0.3) (layer "F.Cu") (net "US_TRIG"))
 (segment (start 58.42 45.72) (end 29.21 45.72) (width 0.3) (layer "F.Cu") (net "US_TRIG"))
 (segment (start 29.21 45.72) (end 29.21 31.75) (width 0.3) (layer "F.Cu") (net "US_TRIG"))
 (via (at 58.42 66.04) (size 0.8) (drill 0.4) (layers "F.Cu" "B.Cu") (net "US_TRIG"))
 (via (at 29.21 31.75) (size 0.8) (drill 0.4) (layers "F.Cu" "B.Cu") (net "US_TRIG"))
 (segment (start 111.76 68.58) (end 58.42 68.58) (width 0.3) (layer "B.Cu") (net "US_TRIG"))
 (segment (start 58.42 68.58) (end 58.42 66.04) (width 0.3) (layer "B.Cu") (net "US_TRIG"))
 (segment (start 29.21 31.75) (end 24.13 31.75) (width 0.3) (layer "B.Cu") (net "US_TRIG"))
 (segment (start 60.96 71.12) (end 60.96 43.18) (width 0.3) (layer "F.Cu") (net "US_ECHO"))
 (segment (start 31.75 43.18) (end 31.75 34.29) (width 0.3) (layer "F.Cu") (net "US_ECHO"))
 (segment (start 60.96 43.18) (end 31.75 43.18) (width 0.3) (layer "F.Cu") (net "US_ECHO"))
 (via (at 60.96 71.12) (size 0.8) (drill 0.4) (layers "F.Cu" "B.Cu") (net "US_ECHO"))
 (via (at 31.75 34.29) (size 0.8) (drill 0.4) (layers "F.Cu" "B.Cu") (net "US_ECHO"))
 (segment (start 31.75 34.29) (end 24.13 34.29) (width 0.3) (layer "B.Cu") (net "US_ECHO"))
 (segment (start 111.76 71.12) (end 60.96 71.12) (width 0.3) (layer "B.Cu") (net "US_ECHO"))
 (segment (start 41.91 66.04) (end 41.91 60.96) (width 0.3) (layer "F.Cu") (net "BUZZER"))
 (segment (start 41.91 60.96) (end 29.21 60.96) (width 0.3) (layer "F.Cu") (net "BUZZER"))
 (segment (start 29.21 60.96) (end 29.21 48.26) (width 0.3) (layer "F.Cu") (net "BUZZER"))
 (segment (start 44.45 66.04) (end 41.91 66.04) (width 0.3) (layer "F.Cu") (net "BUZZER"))
 (via (at 29.21 48.26) (size 0.8) (drill 0.4) (layers "F.Cu" "B.Cu") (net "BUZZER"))
 (via (at 44.45 66.04) (size 0.8) (drill 0.4) (layers "F.Cu" "B.Cu") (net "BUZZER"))
 (segment (start 26.67 48.26) (end 26.67 36.83) (width 0.3) (layer "B.Cu") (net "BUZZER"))
 (segment (start 55.88 77.47) (end 44.45 77.47) (width 0.3) (layer "B.Cu") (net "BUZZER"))
 (segment (start 29.21 48.26) (end 26.67 48.26) (width 0.3) (layer "B.Cu") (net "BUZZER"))
 (segment (start 26.67 36.83) (end 24.13 36.83) (width 0.3) (layer "B.Cu") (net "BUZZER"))
 (segment (start 44.45 77.47) (end 44.45 66.04) (width 0.3) (layer "B.Cu") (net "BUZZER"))
 (segment (start 34.29 40.64) (end 34.29 31.75) (width 0.3) (layer "F.Cu") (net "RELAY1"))
 (segment (start 34.29 31.75) (end 31.75 31.75) (width 0.3) (layer "F.Cu") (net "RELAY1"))
 (segment (start 63.5 40.64) (end 34.29 40.64) (width 0.3) (layer "F.Cu") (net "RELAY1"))
 (segment (start 63.5 50.8) (end 63.5 40.64) (width 0.3) (layer "F.Cu") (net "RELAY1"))
 (segment (start 31.75 31.75) (end 31.75 29.21) (width 0.3) (layer "F.Cu") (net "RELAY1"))
 (segment (start 87.63 50.8) (end 63.5 50.8) (width 0.3) (layer "F.Cu") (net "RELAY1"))
 (segment (start 31.75 29.21) (end 29.21 29.21) (width 0.3) (layer "F.Cu") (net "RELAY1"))
 (via (at 29.21 29.21) (size 0.8) (drill 0.4) (layers "F.Cu" "B.Cu") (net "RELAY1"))
 (segment (start 29.21 29.21) (end 21.59 29.21) (width 0.3) (layer "B.Cu") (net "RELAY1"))
 (segment (start 21.59 29.21) (end 21.59 39.37) (width 0.3) (layer "B.Cu") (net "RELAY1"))
 (segment (start 21.59 39.37) (end 24.13 39.37) (width 0.3) (layer "B.Cu") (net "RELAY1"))
 (segment (start 66.04 38.1) (end 36.83 38.1) (width 0.3) (layer "F.Cu") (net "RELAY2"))
 (segment (start 66.04 48.26) (end 66.04 38.1) (width 0.3) (layer "F.Cu") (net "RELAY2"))
 (segment (start 87.63 48.26) (end 66.04 48.26) (width 0.3) (layer "F.Cu") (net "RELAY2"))
 (segment (start 36.83 29.21) (end 34.29 29.21) (width 0.3) (layer "F.Cu") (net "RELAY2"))
 (segment (start 34.29 29.21) (end 34.29 26.67) (width 0.3) (layer "F.Cu") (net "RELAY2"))
 (segment (start 36.83 38.1) (end 36.83 29.21) (width 0.3) (layer "F.Cu") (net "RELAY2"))
 (segment (start 34.29 26.67) (end 29.21 26.67) (width 0.3) (layer "F.Cu") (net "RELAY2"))
 (via (at 29.21 26.67) (size 0.8) (drill 0.4) (layers "F.Cu" "B.Cu") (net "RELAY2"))
 (segment (start 24.13 41.91) (end 24.13 48.26) (width 0.3) (layer "B.Cu") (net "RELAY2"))
 (segment (start 29.21 26.67) (end 19.05 26.67) (width 0.3) (layer "B.Cu") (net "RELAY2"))
 (segment (start 19.05 41.91) (end 24.13 41.91) (width 0.3) (layer "B.Cu") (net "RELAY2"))
 (segment (start 19.05 26.67) (end 19.05 41.91) (width 0.3) (layer "B.Cu") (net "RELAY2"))
 (segment (start 31.75 48.26) (end 31.75 50.8) (width 0.3) (layer "B.Cu") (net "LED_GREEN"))
 (segment (start 31.75 50.8) (end 24.13 50.8) (width 0.3) (layer "B.Cu") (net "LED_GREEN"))
 (segment (start 55.88 48.26) (end 31.75 48.26) (width 0.3) (layer "B.Cu") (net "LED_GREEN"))
 (segment (start 34.29 50.8) (end 34.29 53.34) (width 0.3) (layer "B.Cu") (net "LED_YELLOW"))
 (segment (start 34.29 53.34) (end 24.13 53.34) (width 0.3) (layer "B.Cu") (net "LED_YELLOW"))
 (segment (start 55.88 50.8) (end 34.29 50.8) (width 0.3) (layer "B.Cu") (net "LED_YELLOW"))
 (segment (start 36.83 53.34) (end 36.83 55.88) (width 0.3) (layer "B.Cu") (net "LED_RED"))
 (segment (start 55.88 53.34) (end 36.83 53.34) (width 0.3) (layer "B.Cu") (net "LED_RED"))
 (segment (start 36.83 55.88) (end 24.13 55.88) (width 0.3) (layer "B.Cu") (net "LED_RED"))
 (segment (start 39.37 63.5) (end 24.13 63.5) (width 0.3) (layer "B.Cu") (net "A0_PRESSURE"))
 (segment (start 29.21 73.66) (end 29.21 71.12) (width 0.3) (layer "F.Cu") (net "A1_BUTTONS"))
 (segment (start 41.91 73.66) (end 29.21 73.66) (width 0.3) (layer "F.Cu") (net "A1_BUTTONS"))
 (segment (start 46.99 71.12) (end 41.91 71.12) (width 0.3) (layer "F.Cu") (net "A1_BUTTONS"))
 (segment (start 41.91 71.12) (end 41.91 73.66) (width 0.3) (layer "F.Cu") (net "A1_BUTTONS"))
 (via (at 29.21 71.12) (size 0.8) (drill 0.4) (layers "F.Cu" "B.Cu") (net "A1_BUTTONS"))
 (via (at 46.99 71.12) (size 0.8) (drill 0.4) (layers "F.Cu" "B.Cu") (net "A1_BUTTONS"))
 (segment (start 29.21 71.12) (end 26.67 71.12) (width 0.3) (layer "B.Cu") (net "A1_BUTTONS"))
 (segment (start 26.67 66.04) (end 24.13 66.04) (width 0.3) (layer "B.Cu") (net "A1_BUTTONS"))
 (segment (start 55.88 66.04) (end 46.99 66.04) (width 0.3) (layer "B.Cu") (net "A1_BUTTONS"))
 (segment (start 26.67 71.12) (end 26.67 66.04) (width 0.3) (layer "B.Cu") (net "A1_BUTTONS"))
 (segment (start 46.99 66.04) (end 46.99 71.12) (width 0.3) (layer "B.Cu") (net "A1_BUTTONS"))
 (segment (start 44.45 60.96) (end 44.45 58.42) (width 0.8) (layer "B.Cu") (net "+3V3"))
 (segment (start 44.45 58.42) (end 19.05 58.42) (width 0.8) (layer "B.Cu") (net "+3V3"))
 (segment (start 58.42 63.5) (end 58.42 60.96) (width 0.8) (layer "B.Cu") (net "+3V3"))
 (segment (start 72.39 16.51) (end 72.39 63.5) (width 0.8) (layer "B.Cu") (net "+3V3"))
 (segment (start 58.42 60.96) (end 44.45 60.96) (width 0.8) (layer "B.Cu") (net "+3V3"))
 (segment (start 19.05 58.42) (end 19.05 63.5) (width 0.8) (layer "B.Cu") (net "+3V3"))
 (segment (start 19.05 63.5) (end 21.59 63.5) (width 0.8) (layer "B.Cu") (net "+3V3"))
 (segment (start 114.3 53.34) (end 114.3 63.5) (width 0.8) (layer "B.Cu") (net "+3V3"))
 (segment (start 21.59 68.58) (end 24.13 68.58) (width 0.8) (layer "B.Cu") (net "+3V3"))
 (segment (start 114.3 63.5) (end 58.42 63.5) (width 0.8) (layer "B.Cu") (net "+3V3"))
 (segment (start 21.59 63.5) (end 21.59 68.58) (width 0.8) (layer "B.Cu") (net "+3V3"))
 (segment (start 111.76 53.34) (end 114.3 53.34) (width 0.8) (layer "B.Cu") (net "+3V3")))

